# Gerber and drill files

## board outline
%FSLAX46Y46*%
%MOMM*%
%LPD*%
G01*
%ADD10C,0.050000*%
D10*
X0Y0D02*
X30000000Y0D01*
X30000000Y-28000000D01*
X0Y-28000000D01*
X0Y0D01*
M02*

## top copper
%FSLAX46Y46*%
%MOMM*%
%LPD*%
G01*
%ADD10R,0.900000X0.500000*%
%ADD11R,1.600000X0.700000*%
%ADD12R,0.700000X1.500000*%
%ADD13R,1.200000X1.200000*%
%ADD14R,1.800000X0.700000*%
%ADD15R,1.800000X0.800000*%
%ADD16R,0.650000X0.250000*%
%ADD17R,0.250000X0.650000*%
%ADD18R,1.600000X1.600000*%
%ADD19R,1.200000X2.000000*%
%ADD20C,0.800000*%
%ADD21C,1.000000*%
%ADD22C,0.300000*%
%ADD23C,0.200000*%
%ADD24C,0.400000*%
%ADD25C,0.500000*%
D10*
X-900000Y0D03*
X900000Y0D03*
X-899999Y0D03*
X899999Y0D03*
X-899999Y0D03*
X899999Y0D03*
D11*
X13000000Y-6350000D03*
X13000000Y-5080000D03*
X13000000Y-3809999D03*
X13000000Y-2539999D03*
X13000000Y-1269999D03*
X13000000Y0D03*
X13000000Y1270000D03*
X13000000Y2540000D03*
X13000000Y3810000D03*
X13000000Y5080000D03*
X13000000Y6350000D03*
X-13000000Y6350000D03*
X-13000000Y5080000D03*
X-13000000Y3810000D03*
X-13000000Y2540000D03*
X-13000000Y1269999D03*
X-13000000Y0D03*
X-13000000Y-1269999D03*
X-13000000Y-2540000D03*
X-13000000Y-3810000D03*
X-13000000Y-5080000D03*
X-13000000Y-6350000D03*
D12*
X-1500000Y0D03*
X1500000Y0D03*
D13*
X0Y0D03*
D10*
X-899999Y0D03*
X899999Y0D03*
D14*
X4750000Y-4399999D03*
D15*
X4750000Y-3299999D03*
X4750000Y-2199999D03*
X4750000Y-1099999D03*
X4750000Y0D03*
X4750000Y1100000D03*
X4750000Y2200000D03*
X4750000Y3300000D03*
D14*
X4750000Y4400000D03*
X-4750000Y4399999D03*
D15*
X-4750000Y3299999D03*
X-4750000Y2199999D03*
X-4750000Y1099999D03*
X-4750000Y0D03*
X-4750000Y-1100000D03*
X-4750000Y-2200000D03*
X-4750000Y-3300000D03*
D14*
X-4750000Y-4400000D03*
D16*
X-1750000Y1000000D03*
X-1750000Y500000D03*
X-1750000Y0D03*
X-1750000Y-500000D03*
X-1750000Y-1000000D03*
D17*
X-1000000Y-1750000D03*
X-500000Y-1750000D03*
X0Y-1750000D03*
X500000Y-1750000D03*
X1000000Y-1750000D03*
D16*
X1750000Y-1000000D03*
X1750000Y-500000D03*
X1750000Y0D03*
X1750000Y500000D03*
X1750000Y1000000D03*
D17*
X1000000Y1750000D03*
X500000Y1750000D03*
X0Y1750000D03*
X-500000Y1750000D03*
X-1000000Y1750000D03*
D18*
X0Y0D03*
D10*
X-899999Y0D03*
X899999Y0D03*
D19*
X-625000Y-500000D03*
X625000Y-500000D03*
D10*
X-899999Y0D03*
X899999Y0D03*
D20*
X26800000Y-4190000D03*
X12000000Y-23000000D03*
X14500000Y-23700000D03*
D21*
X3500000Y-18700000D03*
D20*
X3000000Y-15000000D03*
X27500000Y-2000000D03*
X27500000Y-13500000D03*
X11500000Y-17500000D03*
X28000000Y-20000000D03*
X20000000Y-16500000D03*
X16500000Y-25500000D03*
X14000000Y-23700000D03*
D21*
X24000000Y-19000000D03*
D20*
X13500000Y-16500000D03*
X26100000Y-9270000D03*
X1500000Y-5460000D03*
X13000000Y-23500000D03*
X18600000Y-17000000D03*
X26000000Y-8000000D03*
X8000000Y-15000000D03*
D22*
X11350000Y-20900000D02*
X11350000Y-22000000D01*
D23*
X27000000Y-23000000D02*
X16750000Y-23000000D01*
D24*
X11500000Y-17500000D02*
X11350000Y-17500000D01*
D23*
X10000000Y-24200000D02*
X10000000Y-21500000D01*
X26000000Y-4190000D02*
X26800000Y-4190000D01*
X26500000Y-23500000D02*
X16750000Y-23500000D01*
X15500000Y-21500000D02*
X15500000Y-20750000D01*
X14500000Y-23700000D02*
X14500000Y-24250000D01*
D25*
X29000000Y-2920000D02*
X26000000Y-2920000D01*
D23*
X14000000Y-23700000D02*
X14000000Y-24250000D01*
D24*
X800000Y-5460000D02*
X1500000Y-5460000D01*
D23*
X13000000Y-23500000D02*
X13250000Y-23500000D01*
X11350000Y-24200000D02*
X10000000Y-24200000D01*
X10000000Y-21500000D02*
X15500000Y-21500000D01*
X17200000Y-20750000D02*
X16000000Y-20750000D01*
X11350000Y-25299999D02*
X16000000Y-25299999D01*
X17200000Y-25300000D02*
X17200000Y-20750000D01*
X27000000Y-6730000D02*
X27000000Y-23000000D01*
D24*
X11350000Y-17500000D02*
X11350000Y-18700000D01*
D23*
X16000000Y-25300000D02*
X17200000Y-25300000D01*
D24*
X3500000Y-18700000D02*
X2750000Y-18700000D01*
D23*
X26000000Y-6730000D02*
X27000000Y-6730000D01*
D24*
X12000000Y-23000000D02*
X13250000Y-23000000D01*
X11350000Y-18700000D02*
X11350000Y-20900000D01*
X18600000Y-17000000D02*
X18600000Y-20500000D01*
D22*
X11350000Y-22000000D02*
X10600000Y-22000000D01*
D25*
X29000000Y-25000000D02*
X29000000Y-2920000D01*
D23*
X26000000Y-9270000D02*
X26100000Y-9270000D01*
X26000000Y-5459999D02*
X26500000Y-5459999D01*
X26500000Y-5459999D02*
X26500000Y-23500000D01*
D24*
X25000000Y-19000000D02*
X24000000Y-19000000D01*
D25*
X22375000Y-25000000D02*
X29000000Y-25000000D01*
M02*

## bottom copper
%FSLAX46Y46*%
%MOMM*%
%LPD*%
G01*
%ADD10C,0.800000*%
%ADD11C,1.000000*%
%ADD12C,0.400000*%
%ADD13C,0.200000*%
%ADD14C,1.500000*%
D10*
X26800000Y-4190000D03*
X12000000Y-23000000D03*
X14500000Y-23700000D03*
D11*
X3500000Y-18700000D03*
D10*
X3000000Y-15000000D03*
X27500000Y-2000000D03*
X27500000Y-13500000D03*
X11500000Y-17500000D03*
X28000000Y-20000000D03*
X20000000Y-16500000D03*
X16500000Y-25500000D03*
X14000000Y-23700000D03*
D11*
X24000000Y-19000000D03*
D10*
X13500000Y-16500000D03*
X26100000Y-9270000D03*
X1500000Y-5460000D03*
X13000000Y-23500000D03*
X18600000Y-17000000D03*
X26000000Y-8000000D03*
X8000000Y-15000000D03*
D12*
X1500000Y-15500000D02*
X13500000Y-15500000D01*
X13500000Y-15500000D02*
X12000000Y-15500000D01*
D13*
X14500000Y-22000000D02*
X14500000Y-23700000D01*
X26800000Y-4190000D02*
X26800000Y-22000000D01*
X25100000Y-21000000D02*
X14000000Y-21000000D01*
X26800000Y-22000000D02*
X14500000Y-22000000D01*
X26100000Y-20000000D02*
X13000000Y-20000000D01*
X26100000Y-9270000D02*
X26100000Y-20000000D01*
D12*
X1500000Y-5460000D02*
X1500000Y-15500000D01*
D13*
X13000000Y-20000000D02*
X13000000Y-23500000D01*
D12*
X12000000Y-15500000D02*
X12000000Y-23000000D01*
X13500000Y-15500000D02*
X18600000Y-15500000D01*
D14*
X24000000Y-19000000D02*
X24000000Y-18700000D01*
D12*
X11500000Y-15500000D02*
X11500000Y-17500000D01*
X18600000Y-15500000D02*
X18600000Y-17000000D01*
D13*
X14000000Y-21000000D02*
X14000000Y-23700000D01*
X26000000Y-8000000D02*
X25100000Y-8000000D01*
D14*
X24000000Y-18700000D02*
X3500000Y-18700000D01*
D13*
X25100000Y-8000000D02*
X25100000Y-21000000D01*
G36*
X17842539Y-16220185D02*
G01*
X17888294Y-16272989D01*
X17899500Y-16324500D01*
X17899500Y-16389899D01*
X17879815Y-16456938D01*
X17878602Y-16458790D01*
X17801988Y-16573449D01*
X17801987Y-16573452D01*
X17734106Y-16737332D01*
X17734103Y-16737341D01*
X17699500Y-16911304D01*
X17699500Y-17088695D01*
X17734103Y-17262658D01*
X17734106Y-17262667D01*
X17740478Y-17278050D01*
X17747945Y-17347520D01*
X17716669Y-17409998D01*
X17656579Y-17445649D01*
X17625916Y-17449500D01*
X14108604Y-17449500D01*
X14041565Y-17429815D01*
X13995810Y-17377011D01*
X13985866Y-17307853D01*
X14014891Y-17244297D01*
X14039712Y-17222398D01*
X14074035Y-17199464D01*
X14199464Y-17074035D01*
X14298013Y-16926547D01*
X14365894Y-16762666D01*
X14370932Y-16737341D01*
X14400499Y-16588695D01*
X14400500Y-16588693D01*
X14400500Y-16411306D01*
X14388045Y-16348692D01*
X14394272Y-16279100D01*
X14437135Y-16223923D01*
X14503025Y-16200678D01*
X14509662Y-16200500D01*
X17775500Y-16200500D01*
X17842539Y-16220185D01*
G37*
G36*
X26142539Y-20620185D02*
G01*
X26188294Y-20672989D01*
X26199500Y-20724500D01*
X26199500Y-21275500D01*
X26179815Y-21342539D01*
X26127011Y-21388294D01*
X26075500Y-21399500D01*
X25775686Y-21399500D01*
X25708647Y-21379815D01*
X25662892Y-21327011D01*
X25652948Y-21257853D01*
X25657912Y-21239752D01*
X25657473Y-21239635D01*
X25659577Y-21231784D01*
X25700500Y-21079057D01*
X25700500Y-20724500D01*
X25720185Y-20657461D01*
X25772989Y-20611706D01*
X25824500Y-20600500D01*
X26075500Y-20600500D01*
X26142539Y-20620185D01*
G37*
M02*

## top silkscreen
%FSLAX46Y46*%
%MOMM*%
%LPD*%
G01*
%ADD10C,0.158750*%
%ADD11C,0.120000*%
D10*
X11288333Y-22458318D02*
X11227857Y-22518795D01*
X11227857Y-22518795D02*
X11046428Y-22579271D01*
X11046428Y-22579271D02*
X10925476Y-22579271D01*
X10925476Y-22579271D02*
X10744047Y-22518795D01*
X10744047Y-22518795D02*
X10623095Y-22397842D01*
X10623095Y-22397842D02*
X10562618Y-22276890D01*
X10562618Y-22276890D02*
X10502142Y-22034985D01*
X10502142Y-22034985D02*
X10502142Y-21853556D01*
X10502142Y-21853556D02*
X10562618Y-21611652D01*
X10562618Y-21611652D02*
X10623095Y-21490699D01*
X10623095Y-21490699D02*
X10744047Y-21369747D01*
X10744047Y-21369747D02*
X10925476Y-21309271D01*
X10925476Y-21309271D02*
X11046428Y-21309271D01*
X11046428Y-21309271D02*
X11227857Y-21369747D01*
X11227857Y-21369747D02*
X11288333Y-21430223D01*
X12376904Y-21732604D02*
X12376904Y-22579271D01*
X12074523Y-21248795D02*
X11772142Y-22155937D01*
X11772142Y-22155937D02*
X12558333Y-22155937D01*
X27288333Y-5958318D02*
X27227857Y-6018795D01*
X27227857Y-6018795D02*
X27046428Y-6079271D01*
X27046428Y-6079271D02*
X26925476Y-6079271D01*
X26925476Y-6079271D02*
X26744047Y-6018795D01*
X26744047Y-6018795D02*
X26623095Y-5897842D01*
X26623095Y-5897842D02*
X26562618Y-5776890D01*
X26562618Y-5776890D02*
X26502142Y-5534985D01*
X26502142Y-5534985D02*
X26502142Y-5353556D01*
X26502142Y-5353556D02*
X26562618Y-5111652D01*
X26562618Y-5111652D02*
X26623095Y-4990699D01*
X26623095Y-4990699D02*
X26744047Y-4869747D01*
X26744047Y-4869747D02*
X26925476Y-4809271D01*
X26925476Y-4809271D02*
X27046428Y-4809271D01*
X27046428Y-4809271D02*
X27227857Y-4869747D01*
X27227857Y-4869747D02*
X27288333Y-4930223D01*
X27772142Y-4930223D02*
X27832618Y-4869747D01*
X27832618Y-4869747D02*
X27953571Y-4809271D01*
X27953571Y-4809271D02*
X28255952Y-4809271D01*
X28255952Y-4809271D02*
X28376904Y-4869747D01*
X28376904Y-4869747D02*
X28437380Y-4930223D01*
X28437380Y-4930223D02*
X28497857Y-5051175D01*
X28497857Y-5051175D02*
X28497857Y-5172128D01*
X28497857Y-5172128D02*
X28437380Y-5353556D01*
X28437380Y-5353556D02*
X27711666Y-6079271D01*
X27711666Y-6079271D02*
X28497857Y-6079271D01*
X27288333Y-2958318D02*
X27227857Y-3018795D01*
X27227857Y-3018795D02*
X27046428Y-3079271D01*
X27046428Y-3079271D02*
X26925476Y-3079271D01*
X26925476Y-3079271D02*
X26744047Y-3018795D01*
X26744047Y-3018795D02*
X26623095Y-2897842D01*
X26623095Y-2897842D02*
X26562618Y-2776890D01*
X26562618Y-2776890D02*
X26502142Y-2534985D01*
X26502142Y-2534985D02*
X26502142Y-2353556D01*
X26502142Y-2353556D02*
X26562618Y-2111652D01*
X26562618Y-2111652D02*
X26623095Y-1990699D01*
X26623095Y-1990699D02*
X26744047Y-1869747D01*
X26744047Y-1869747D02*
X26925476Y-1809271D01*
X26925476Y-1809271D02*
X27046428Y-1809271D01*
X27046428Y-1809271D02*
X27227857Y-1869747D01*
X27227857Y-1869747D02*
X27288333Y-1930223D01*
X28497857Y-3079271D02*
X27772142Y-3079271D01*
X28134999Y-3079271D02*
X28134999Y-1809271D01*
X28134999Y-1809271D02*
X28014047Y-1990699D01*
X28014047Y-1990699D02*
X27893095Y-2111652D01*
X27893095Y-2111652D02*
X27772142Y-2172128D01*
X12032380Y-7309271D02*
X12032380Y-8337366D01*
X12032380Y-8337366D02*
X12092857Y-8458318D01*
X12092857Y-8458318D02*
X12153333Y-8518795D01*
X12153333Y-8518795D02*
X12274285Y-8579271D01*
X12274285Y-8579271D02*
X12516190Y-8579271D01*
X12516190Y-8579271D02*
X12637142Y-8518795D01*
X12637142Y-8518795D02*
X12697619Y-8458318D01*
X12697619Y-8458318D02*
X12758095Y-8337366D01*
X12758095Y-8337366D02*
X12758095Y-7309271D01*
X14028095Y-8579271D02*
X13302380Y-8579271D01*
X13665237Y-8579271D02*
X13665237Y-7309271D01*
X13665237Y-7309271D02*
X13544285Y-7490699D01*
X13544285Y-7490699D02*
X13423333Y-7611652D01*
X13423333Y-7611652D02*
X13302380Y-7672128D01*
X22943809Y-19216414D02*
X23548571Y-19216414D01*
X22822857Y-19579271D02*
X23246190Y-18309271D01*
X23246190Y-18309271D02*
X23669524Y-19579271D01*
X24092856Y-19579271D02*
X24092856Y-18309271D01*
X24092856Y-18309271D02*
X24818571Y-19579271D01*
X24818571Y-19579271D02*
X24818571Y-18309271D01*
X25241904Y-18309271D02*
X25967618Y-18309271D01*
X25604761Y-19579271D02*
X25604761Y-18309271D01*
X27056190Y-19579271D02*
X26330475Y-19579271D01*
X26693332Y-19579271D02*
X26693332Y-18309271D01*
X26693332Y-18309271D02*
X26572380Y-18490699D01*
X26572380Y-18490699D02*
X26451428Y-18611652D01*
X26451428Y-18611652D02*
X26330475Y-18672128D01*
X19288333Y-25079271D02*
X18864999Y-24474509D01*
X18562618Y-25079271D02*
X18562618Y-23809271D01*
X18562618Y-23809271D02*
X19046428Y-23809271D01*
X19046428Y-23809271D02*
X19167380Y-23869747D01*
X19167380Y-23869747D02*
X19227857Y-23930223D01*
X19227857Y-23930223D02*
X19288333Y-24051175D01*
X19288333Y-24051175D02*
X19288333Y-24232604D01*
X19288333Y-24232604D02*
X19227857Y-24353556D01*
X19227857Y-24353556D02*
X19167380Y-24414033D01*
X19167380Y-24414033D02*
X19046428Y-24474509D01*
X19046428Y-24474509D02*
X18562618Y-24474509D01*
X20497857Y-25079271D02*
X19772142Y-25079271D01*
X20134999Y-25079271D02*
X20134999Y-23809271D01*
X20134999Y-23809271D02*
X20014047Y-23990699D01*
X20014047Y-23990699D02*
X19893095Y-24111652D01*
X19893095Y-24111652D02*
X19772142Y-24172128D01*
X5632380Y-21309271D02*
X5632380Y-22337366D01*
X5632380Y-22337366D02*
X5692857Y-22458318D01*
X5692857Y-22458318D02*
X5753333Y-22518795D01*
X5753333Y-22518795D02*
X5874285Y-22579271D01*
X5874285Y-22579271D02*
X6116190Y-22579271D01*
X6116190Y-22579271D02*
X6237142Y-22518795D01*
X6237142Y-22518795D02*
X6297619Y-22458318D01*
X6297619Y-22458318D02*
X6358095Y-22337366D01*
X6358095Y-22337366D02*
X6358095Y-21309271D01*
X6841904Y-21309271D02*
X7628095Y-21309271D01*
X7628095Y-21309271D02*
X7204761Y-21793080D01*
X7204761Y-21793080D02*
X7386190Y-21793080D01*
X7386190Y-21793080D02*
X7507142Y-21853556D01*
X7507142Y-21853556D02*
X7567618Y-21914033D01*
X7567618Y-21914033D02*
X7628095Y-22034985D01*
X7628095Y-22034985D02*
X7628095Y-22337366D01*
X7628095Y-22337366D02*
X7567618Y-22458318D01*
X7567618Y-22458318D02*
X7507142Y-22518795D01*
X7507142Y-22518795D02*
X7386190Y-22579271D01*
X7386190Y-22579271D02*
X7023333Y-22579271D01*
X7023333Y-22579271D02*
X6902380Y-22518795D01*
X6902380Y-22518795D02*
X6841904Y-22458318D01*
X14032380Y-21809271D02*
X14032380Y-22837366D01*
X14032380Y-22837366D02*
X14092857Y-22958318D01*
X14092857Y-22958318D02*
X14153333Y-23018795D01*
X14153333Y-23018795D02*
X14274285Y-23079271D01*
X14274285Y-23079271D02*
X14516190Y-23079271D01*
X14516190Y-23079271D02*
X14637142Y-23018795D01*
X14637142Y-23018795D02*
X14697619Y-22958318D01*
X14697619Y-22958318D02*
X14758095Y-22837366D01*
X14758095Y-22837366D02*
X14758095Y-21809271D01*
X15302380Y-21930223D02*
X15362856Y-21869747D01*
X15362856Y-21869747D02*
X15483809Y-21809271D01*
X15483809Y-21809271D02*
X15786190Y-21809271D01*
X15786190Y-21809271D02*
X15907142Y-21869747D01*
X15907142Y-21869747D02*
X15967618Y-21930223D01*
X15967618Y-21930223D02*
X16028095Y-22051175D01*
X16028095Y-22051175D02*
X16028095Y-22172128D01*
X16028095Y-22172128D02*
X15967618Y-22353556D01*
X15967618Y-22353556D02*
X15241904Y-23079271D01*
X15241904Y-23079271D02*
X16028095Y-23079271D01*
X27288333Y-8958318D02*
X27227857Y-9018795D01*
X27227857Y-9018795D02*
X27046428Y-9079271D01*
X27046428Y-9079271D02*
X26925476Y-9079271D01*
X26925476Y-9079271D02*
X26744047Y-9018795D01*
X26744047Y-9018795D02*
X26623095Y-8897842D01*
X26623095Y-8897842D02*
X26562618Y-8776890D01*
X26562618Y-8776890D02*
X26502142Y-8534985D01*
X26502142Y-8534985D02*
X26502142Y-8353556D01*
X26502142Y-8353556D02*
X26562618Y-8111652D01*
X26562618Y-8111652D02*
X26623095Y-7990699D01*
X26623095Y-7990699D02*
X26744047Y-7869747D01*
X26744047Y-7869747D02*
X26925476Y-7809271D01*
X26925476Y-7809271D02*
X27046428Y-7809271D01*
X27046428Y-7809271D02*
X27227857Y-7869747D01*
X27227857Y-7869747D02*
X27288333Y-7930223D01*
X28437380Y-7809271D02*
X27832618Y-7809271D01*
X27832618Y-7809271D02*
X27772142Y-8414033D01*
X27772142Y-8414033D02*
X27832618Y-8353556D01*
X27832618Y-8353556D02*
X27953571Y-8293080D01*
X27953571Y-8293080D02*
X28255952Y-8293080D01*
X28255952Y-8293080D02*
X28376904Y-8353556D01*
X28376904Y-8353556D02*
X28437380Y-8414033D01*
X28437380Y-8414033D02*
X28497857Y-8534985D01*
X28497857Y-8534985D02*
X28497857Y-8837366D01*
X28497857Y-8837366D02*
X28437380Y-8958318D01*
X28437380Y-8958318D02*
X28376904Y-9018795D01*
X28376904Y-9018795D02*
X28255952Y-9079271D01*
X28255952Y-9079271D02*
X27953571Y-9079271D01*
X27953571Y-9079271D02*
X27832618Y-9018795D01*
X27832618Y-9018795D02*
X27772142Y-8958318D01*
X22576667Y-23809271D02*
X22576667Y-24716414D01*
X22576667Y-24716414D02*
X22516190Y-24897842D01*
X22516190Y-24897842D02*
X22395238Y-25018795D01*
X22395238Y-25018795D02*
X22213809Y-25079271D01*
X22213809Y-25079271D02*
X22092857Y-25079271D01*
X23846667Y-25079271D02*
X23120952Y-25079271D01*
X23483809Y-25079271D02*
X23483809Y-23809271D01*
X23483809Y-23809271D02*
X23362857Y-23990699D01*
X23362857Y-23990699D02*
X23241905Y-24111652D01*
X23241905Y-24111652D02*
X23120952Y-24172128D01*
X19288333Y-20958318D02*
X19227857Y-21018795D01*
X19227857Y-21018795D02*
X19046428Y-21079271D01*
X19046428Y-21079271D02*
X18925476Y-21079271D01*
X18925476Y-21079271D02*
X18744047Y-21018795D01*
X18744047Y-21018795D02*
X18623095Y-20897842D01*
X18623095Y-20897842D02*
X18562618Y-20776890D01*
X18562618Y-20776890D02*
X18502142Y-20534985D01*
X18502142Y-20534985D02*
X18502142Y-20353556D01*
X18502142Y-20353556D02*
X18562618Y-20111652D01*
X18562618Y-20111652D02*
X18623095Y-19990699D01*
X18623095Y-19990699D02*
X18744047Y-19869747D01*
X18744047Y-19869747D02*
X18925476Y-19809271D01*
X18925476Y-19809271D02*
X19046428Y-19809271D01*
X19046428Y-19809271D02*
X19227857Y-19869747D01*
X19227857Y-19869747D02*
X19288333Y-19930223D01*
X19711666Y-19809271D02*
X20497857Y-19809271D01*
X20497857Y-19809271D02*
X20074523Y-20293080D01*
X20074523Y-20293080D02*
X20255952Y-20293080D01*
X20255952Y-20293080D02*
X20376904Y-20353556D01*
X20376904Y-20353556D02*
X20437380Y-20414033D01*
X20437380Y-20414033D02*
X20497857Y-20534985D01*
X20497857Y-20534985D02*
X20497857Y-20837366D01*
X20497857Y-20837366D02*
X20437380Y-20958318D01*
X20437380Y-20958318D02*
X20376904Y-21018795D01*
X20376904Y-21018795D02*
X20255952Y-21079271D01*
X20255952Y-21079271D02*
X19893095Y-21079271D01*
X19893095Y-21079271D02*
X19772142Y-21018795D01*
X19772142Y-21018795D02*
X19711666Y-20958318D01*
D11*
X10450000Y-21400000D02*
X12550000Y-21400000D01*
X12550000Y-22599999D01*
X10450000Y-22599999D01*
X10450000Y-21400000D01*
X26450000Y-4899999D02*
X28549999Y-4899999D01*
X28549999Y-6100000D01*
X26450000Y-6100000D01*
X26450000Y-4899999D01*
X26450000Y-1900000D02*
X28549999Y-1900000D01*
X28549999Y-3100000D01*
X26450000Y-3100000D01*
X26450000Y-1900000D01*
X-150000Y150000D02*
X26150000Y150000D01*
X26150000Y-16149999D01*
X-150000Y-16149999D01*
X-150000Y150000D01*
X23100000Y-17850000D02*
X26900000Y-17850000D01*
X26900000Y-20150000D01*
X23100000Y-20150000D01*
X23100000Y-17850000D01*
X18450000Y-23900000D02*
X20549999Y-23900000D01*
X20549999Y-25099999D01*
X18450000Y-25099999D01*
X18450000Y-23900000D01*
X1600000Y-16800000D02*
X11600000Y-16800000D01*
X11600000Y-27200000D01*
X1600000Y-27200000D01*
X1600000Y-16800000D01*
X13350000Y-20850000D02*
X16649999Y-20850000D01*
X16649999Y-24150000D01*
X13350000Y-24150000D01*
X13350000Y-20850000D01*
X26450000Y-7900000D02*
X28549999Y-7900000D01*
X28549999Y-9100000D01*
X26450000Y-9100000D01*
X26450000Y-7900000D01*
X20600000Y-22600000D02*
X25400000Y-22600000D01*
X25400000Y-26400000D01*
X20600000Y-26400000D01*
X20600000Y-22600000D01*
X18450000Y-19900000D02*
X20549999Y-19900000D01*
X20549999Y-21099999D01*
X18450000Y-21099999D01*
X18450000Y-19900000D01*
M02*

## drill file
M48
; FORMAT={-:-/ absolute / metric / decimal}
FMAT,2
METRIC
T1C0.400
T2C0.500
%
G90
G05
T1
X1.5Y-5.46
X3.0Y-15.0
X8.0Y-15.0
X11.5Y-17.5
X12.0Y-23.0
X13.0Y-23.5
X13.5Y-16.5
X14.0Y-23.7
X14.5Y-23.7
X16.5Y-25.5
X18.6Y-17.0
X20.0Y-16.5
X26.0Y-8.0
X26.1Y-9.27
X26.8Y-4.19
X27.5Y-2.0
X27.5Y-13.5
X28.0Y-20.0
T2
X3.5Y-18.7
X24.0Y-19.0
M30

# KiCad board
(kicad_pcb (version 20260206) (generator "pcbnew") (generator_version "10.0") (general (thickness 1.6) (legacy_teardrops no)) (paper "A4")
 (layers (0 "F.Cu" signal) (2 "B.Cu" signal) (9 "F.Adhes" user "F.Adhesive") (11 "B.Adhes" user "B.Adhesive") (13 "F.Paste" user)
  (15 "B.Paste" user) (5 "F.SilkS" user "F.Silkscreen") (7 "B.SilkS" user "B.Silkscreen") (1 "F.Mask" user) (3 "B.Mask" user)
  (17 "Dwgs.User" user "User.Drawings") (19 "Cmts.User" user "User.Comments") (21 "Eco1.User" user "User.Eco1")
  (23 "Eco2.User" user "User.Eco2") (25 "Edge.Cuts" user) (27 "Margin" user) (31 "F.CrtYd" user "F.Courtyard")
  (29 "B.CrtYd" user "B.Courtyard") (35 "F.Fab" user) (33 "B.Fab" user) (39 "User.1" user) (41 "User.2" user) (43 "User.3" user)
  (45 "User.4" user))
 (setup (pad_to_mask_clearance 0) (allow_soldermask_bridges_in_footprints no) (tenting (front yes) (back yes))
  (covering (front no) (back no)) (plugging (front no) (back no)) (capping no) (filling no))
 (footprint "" (layer "F.Cu") (at 11.5 22)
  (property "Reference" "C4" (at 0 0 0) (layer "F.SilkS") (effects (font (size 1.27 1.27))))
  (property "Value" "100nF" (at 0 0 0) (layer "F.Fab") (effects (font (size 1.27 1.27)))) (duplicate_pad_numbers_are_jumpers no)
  (fp_rect (start -1.05 -0.6) (end 1.05 0.599999) (stroke (width 0.12) (type default)) (fill no) (layer "F.SilkS"))
  (pad "1" smd rect (at -12.4 -22) (size 0.9 0.5) (layers "F.Cu" "F.Mask" "F.Paste") (thermal_bridge_angle 45))
  (pad "2" smd rect (at -10.6 -22) (size 0.9 0.5) (layers "F.Cu" "F.Mask" "F.Paste") (thermal_bridge_angle 45)))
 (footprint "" (layer "F.Cu") (at 27.5 5.5)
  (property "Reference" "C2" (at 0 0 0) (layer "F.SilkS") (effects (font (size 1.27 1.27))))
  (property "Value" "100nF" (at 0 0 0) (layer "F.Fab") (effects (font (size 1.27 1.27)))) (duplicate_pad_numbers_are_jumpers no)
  (fp_rect (start -1.05 -0.600001) (end 1.049999 0.6) (stroke (width 0.12) (type default)) (fill no) (layer "F.SilkS"))
  (pad "1" smd rect (at -28.399999 -5.5) (size 0.9 0.5) (layers "F.Cu" "F.Mask" "F.Paste") (thermal_bridge_angle 45))
  (pad "2" smd rect (at -26.600001 -5.5) (size 0.9 0.5) (layers "F.Cu" "F.Mask" "F.Paste") (thermal_bridge_angle 45)))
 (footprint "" (layer "F.Cu") (at 27.5 2.5)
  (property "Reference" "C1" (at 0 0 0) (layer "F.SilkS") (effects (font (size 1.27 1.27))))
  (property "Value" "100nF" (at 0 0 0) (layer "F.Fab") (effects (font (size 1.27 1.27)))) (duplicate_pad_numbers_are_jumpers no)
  (fp_rect (start -1.05 -0.6) (end 1.049999 0.6) (stroke (width 0.12) (type default)) (fill no) (layer "F.SilkS"))
  (pad "1" smd rect (at -28.399999 -2.5) (size 0.9 0.5) (layers "F.Cu" "F.Mask" "F.Paste") (thermal_bridge_angle 45))
  (pad "2" smd rect (at -26.600001 -2.5) (size 0.9 0.5) (layers "F.Cu" "F.Mask" "F.Paste") (thermal_bridge_angle 45)))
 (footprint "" (layer "F.Cu") (at 13 8)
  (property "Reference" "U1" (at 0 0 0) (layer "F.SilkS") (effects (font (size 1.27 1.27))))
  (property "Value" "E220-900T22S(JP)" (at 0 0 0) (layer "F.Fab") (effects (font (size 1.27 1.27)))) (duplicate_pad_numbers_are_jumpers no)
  (fp_rect (start -13.15 -8.15) (end 13.15 8.149999) (stroke (width 0.12) (type default)) (fill no) (layer "F.SilkS"))
  (pad "1" smd rect (at 0 -1.65) (size 1.6 0.7) (layers "F.Cu" "F.Mask" "F.Paste") (thermal_bridge_angle 45))
  (pad "2" smd rect (at 0 -2.92) (size 1.6 0.7) (layers "F.Cu" "F.Mask" "F.Paste") (thermal_bridge_angle 45))
  (pad "3" smd rect (at 0 -4.190001) (size 1.6 0.7) (layers "F.Cu" "F.Mask" "F.Paste") (thermal_bridge_angle 45))
  (pad "4" smd rect (at 0 -5.460001) (size 1.6 0.7) (layers "F.Cu" "F.Mask" "F.Paste") (thermal_bridge_angle 45))
  (pad "5" smd rect (at 0 -6.730001) (size 1.6 0.7) (layers "F.Cu" "F.Mask" "F.Paste") (thermal_bridge_angle 45))
  (pad "6" smd rect (at 0 -8) (size 1.6 0.7) (layers "F.Cu" "F.Mask" "F.Paste") (thermal_bridge_angle 45))
  (pad "7" smd rect (at 0 -9.27) (size 1.6 0.7) (layers "F.Cu" "F.Mask" "F.Paste") (thermal_bridge_angle 45))
  (pad "8" smd rect (at 0 -10.54) (size 1.6 0.7) (layers "F.Cu" "F.Mask" "F.Paste") (thermal_bridge_angle 45))
  (pad "9" smd rect (at 0 -11.81) (size 1.6 0.7) (layers "F.Cu" "F.Mask" "F.Paste") (thermal_bridge_angle 45))
  (pad "10" smd rect (at 0 -13.08) (size 1.6 0.7) (layers "F.Cu" "F.Mask" "F.Paste") (thermal_bridge_angle 45))
  (pad "11" smd rect (at 0 -14.35) (size 1.6 0.7) (layers "F.Cu" "F.Mask" "F.Paste") (thermal_bridge_angle 45))
  (pad "12" smd rect (at -26 -14.35) (size 1.6 0.7) (layers "F.Cu" "F.Mask" "F.Paste") (thermal_bridge_angle 45))
  (pad "13" smd rect (at -26 -13.08) (size 1.6 0.7) (layers "F.Cu" "F.Mask" "F.Paste") (thermal_bridge_angle 45))
  (pad "14" smd rect (at -26 -11.81) (size 1.6 0.7) (layers "F.Cu" "F.Mask" "F.Paste") (thermal_bridge_angle 45))
  (pad "15" smd rect (at -26 -10.54) (size 1.6 0.7) (layers "F.Cu" "F.Mask" "F.Paste") (thermal_bridge_angle 45))
  (pad "16" smd rect (at -26 -9.269999) (size 1.6 0.7) (layers "F.Cu" "F.Mask" "F.Paste") (thermal_bridge_angle 45))
  (pad "17" smd rect (at -26 -8) (size 1.6 0.7) (layers "F.Cu" "F.Mask" "F.Paste") (thermal_bridge_angle 45))
  (pad "18" smd rect (at -26 -6.730001) (size 1.6 0.7) (layers "F.Cu" "F.Mask" "F.Paste") (thermal_bridge_angle 45))
  (pad "19" smd rect (at -26 -5.46) (size 1.6 0.7) (layers "F.Cu" "F.Mask" "F.Paste") (thermal_bridge_angle 45))
  (pad "20" smd rect (at -26 -4.19) (size 1.6 0.7) (layers "F.Cu" "F.Mask" "F.Paste") (thermal_bridge_angle 45))
  (pad "21" smd rect (at -26 -2.92) (size 1.6 0.7) (layers "F.Cu" "F.Mask" "F.Paste") (thermal_bridge_angle 45))
  (pad "22" smd rect (at -26 -1.65) (size 1.6 0.7) (layers "F.Cu" "F.Mask" "F.Paste") (thermal_bridge_angle 45)))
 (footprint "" (layer "F.Cu") (at 25 19)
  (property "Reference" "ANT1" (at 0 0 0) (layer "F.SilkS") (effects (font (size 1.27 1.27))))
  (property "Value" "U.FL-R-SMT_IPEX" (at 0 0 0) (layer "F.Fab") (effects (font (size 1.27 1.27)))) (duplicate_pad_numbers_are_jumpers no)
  (fp_rect (start -1.9 -1.15) (end 1.9 1.15) (stroke (width 0.12) (type default)) (fill no) (layer "F.SilkS"))
  (pad "G1" smd rect (at -26.5 -19) (size 0.7 1.5) (layers "F.Cu" "F.Mask" "F.Paste") (thermal_bridge_angle 45))
  (pad "G2" smd rect (at -23.5 -19) (size 0.7 1.5) (layers "F.Cu" "F.Mask" "F.Paste") (thermal_bridge_angle 45))
  (pad "S" smd rect (at -25 -19) (size 1.2 1.2) (layers "F.Cu" "F.Mask" "F.Paste") (thermal_bridge_angle 45)))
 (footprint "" (layer "F.Cu") (at 19.5 24.5)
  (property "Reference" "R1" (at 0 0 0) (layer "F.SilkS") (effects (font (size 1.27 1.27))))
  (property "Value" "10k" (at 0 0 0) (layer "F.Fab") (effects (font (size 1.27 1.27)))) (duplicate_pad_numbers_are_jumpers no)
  (fp_rect (start -1.05 -0.6) (end 1.049999 0.599999) (stroke (width 0.12) (type default)) (fill no) (layer "F.SilkS"))
  (pad "1" smd rect (at -20.399999 -24.5) (size 0.9 0.5) (layers "F.Cu" "F.Mask" "F.Paste") (thermal_bridge_angle 45))
  (pad "2" smd rect (at -18.600001 -24.5) (size 0.9 0.5) (layers "F.Cu" "F.Mask" "F.Paste") (thermal_bridge_angle 45)))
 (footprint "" (layer "F.Cu") (at 6.6 22)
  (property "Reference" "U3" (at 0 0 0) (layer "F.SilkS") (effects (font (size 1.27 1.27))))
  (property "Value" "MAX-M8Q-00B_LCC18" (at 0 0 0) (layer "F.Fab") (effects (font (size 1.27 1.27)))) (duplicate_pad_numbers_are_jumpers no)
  (fp_rect (start -5 -5.2) (end 5 5.2) (stroke (width 0.12) (type default)) (fill no) (layer "F.SilkS"))
  (pad "1" smd rect (at -1.85 -17.600001) (size 1.8 0.7) (layers "F.Cu" "F.Mask" "F.Paste") (thermal_bridge_angle 45))
  (pad "2" smd rect (at -1.85 -18.700001) (size 1.8 0.8) (layers "F.Cu" "F.Mask" "F.Paste") (thermal_bridge_angle 45))
  (pad "3" smd rect (at -1.85 -19.800001) (size 1.8 0.8) (layers "F.Cu" "F.Mask" "F.Paste") (thermal_bridge_angle 45))
  (pad "4" smd rect (at -1.85 -20.900001) (size 1.8 0.8) (layers "F.Cu" "F.Mask" "F.Paste") (thermal_bridge_angle 45))
  (pad "5" smd rect (at -1.85 -22) (size 1.8 0.8) (layers "F.Cu" "F.Mask" "F.Paste") (thermal_bridge_angle 45))
  (pad "6" smd rect (at -1.85 -23.1) (size 1.8 0.8) (layers "F.Cu" "F.Mask" "F.Paste") (thermal_bridge_angle 45))
  (pad "7" smd rect (at -1.85 -24.2) (size 1.8 0.8) (layers "F.Cu" "F.Mask" "F.Paste") (thermal_bridge_angle 45))
  (pad "8" smd rect (at -1.85 -25.3) (size 1.8 0.8) (layers "F.Cu" "F.Mask" "F.Paste") (thermal_bridge_angle 45))
  (pad "9" smd rect (at -1.85 -26.4) (size 1.8 0.7) (layers "F.Cu" "F.Mask" "F.Paste") (thermal_bridge_angle 45))
  (pad "10" smd rect (at -11.35 -26.399999) (size 1.8 0.7) (layers "F.Cu" "F.Mask" "F.Paste") (thermal_bridge_angle 45))
  (pad "11" smd rect (at -11.35 -25.299999) (size 1.8 0.8) (layers "F.Cu" "F.Mask" "F.Paste") (thermal_bridge_angle 45))
  (pad "12" smd rect (at -11.35 -24.199999) (size 1.8 0.8) (layers "F.Cu" "F.Mask" "F.Paste") (thermal_bridge_angle 45))
  (pad "13" smd rect (at -11.35 -23.099999) (size 1.8 0.8) (layers "F.Cu" "F.Mask" "F.Paste") (thermal_bridge_angle 45))
  (pad "14" smd rect (at -11.35 -22) (size 1.8 0.8) (layers "F.Cu" "F.Mask" "F.Paste") (thermal_bridge_angle 45))
  (pad "15" smd rect (at -11.35 -20.9) (size 1.8 0.8) (layers "F.Cu" "F.Mask" "F.Paste") (thermal_bridge_angle 45))
  (pad "16" smd rect (at -11.35 -19.8) (size 1.8 0.8) (layers "F.Cu" "F.Mask" "F.Paste") (thermal_bridge_angle 45))
  (pad "17" smd rect (at -11.35 -18.7) (size 1.8 0.8) (layers "F.Cu" "F.Mask" "F.Paste") (thermal_bridge_angle 45))
  (pad "18" smd rect (at -11.35 -17.6) (size 1.8 0.7) (layers "F.Cu" "F.Mask" "F.Paste") (thermal_bridge_angle 45)))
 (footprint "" (layer "F.Cu") (at 15 22.5)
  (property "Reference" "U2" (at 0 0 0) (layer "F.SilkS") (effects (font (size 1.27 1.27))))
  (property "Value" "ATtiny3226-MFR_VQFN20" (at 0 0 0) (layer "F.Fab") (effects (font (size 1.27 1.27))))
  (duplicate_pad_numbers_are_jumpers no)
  (fp_rect (start -1.65 -1.65) (end 1.649999 1.65) (stroke (width 0.12) (type default)) (fill no) (layer "F.SilkS"))
  (pad "1" smd rect (at -16.75 -23.5) (size 0.65 0.25) (layers "F.Cu" "F.Mask" "F.Paste") (thermal_bridge_angle 45))
  (pad "2" smd rect (at -16.75 -23) (size 0.65 0.25) (layers "F.Cu" "F.Mask" "F.Paste") (thermal_bridge_angle 45))
  (pad "3" smd rect (at -16.75 -22.5) (size 0.65 0.25) (layers "F.Cu" "F.Mask" "F.Paste") (thermal_bridge_angle 45))
  (pad "4" smd rect (at -16.75 -22) (size 0.65 0.25) (layers "F.Cu" "F.Mask" "F.Paste") (thermal_bridge_angle 45))
  (pad "5" smd rect (at -16.75 -21.5) (size 0.65 0.25) (layers "F.Cu" "F.Mask" "F.Paste") (thermal_bridge_angle 45))
  (pad "6" smd rect (at -16 -20.75) (size 0.25 0.65) (layers "F.Cu" "F.Mask" "F.Paste") (thermal_bridge_angle 45))
  (pad "7" smd rect (at -15.5 -20.75) (size 0.25 0.65) (layers "F.Cu" "F.Mask" "F.Paste") (thermal_bridge_angle 45))
  (pad "8" smd rect (at -15 -20.75) (size 0.25 0.65) (layers "F.Cu" "F.Mask" "F.Paste") (thermal_bridge_angle 45))
  (pad "9" smd rect (at -14.5 -20.75) (size 0.25 0.65) (layers "F.Cu" "F.Mask" "F.Paste") (thermal_bridge_angle 45))
  (pad "10" smd rect (at -14 -20.75) (size 0.25 0.65) (layers "F.Cu" "F.Mask" "F.Paste") (thermal_bridge_angle 45))
  (pad "11" smd rect (at -13.25 -21.5) (size 0.65 0.25) (layers "F.Cu" "F.Mask" "F.Paste") (thermal_bridge_angle 45))
  (pad "12" smd rect (at -13.25 -22) (size 0.65 0.25) (layers "F.Cu" "F.Mask" "F.Paste") (thermal_bridge_angle 45))
  (pad "13" smd rect (at -13.25 -22.5) (size 0.65 0.25) (layers "F.Cu" "F.Mask" "F.Paste") (thermal_bridge_angle 45))
  (pad "14" smd rect (at -13.25 -23) (size 0.65 0.25) (layers "F.Cu" "F.Mask" "F.Paste") (thermal_bridge_angle 45))
  (pad "15" smd rect (at -13.25 -23.5) (size 0.65 0.25) (layers "F.Cu" "F.Mask" "F.Paste") (thermal_bridge_angle 45))
  (pad "16" smd rect (at -14 -24.25) (size 0.25 0.65) (layers "F.Cu" "F.Mask" "F.Paste") (thermal_bridge_angle 45))
  (pad "17" smd rect (at -14.5 -24.25) (size 0.25 0.65) (layers "F.Cu" "F.Mask" "F.Paste") (thermal_bridge_angle 45))
  (pad "18" smd rect (at -15 -24.25) (size 0.25 0.65) (layers "F.Cu" "F.Mask" "F.Paste") (thermal_bridge_angle 45))
  (pad "19" smd rect (at -15.5 -24.25) (size 0.25 0.65) (layers "F.Cu" "F.Mask" "F.Paste") (thermal_bridge_angle 45))
  (pad "20" smd rect (at -16 -24.25) (size 0.25 0.65) (layers "F.Cu" "F.Mask" "F.Paste") (thermal_bridge_angle 45))
  (pad "EP" smd rect (at -15 -22.5) (size 1.6 1.6) (layers "F.Cu" "F.Mask" "F.Paste") (thermal_bridge_angle 45)))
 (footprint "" (layer "F.Cu") (at 27.5 8.5)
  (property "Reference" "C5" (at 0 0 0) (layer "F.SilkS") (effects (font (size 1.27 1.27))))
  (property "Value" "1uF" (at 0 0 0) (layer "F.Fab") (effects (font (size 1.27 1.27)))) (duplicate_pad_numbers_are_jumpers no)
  (fp_rect (start -1.05 -0.6) (end 1.049999 0.6) (stroke (width 0.12) (type default)) (fill no) (layer "F.SilkS"))
  (pad "1" smd rect (at -28.399999 -8.5) (size 0.9 0.5) (layers "F.Cu" "F.Mask" "F.Paste") (thermal_bridge_angle 45))
  (pad "2" smd rect (at -26.600001 -8.5) (size 0.9 0.5) (layers "F.Cu" "F.Mask" "F.Paste") (thermal_bridge_angle 45)))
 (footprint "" (layer "F.Cu") (at 23 24.5)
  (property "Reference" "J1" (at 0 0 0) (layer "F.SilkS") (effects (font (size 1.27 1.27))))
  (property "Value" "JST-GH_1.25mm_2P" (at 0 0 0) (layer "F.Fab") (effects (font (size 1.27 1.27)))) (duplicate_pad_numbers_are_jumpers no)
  (fp_rect (start -2.4 -1.9) (end 2.4 1.9) (stroke (width 0.12) (type default)) (fill no) (layer "F.SilkS"))
  (pad "1" smd rect (at -23.625 -24) (size 1.2 2) (layers "F.Cu" "F.Mask" "F.Paste") (thermal_bridge_angle 45))
  (pad "2" smd rect (at -22.375 -24) (size 1.2 2) (layers "F.Cu" "F.Mask" "F.Paste") (thermal_bridge_angle 45)))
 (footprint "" (layer "F.Cu") (at 19.5 20.5)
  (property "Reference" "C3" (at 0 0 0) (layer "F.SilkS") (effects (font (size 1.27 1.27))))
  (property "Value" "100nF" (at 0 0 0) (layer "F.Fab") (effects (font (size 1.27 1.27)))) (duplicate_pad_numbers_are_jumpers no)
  (fp_rect (start -1.05 -0.6) (end 1.049999 0.599999) (stroke (width 0.12) (type default)) (fill no) (layer "F.SilkS"))
  (pad "1" smd rect (at -20.399999 -20.5) (size 0.9 0.5) (layers "F.Cu" "F.Mask" "F.Paste") (thermal_bridge_angle 45))
  (pad "2" smd rect (at -18.600001 -20.5) (size 0.9 0.5) (layers "F.Cu" "F.Mask" "F.Paste") (thermal_bridge_angle 45)))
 (gr_rect (start 0 0) (end 30 28) (stroke (width 0.05) (type default)) (fill no) (layer "Edge.Cuts"))
 (segment (start 11.35 20.9) (end 11.35 22) (width 0.3) (layer "F.Cu") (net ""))
 (segment (start 27 23) (end 16.75 23) (width 0.2) (layer "F.Cu") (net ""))
 (segment (start 11.5 17.5) (end 11.35 17.5) (width 0.4) (layer "F.Cu") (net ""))
 (segment (start 10 24.2) (end 10 21.5) (width 0.2) (layer "F.Cu") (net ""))
 (segment (start 26 4.19) (end 26.8 4.19) (width 0.2) (layer "F.Cu") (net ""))
 (segment (start 26.5 23.5) (end 16.75 23.5) (width 0.2) (layer "F.Cu") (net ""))
 (segment (start 15.5 21.5) (end 15.5 20.75) (width 0.2) (layer "F.Cu") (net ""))
 (segment (start 14.5 23.7) (end 14.5 24.25) (width 0.2) (layer "F.Cu") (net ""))
 (segment (start 29 2.92) (end 26 2.92) (width 0.5) (layer "F.Cu") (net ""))
 (segment (start 14 23.7) (end 14 24.25) (width 0.2) (layer "F.Cu") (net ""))
 (segment (start 0.8 5.46) (end 1.5 5.46) (width 0.4) (layer "F.Cu") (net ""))
 (segment (start 13 23.5) (end 13.25 23.5) (width 0.2) (layer "F.Cu") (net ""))
 (segment (start 11.35 24.2) (end 10 24.2) (width 0.2) (layer "F.Cu") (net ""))
 (segment (start 10 21.5) (end 15.5 21.5) (width 0.2) (layer "F.Cu") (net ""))
 (segment (start 17.2 20.75) (end 16 20.75) (width 0.2) (layer "F.Cu") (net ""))
 (segment (start 11.35 25.299999) (end 16 25.299999) (width 0.2) (layer "F.Cu") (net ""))
 (segment (start 17.2 25.3) (end 17.2 20.75) (width 0.2) (layer "F.Cu") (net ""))
 (segment (start 27 6.73) (end 27 23) (width 0.2) (layer "F.Cu") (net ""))
 (segment (start 11.35 17.5) (end 11.35 18.7) (width 0.4) (layer "F.Cu") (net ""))
 (segment (start 16 25.3) (end 17.2 25.3) (width 0.2) (layer "F.Cu") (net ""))
 (segment (start 3.5 18.7) (end 2.75 18.7) (width 0.4) (layer "F.Cu") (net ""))
 (segment (start 26 6.73) (end 27 6.73) (width 0.2) (layer "F.Cu") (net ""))
 (segment (start 12 23) (end 13.25 23) (width 0.4) (layer "F.Cu") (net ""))
 (segment (start 11.35 18.7) (end 11.35 20.9) (width 0.4) (layer "F.Cu") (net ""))
 (segment (start 18.6 17) (end 18.6 20.5) (width 0.4) (layer "F.Cu") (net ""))
 (segment (start 11.35 22) (end 10.6 22) (width 0.3) (layer "F.Cu") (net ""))
 (segment (start 29 25) (end 29 2.92) (width 0.5) (layer "F.Cu") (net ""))
 (segment (start 26 9.27) (end 26.1 9.27) (width 0.2) (layer "F.Cu") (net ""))
 (segment (start 26 5.459999) (end 26.5 5.459999) (width 0.2) (layer "F.Cu") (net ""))
 (segment (start 26.5 5.459999) (end 26.5 23.5) (width 0.2) (layer "F.Cu") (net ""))
 (segment (start 25 19) (end 24 19) (width 0.4) (layer "F.Cu") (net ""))
 (segment (start 22.375 25) (end 29 25) (width 0.5) (layer "F.Cu") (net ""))
 (via (at 26.8 4.19) (size 0.8) (drill 0.4) (layers "F.Cu" "B.Cu") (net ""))
 (via (at 12 23) (size 0.8) (drill 0.4) (layers "F.Cu" "B.Cu") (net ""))
 (via (at 14.5 23.7) (size 0.8) (drill 0.4) (layers "F.Cu" "B.Cu") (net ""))
 (via (at 3.5 18.7) (size 1) (drill 0.5) (layers "F.Cu" "B.Cu") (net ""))
 (via (at 3 15) (size 0.8) (drill 0.4) (layers "F.Cu" "B.Cu") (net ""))
 (via (at 27.5 2) (size 0.8) (drill 0.4) (layers "F.Cu" "B.Cu") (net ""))
 (via (at 27.5 13.5) (size 0.8) (drill 0.4) (layers "F.Cu" "B.Cu") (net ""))
 (via (at 11.5 17.5) (size 0.8) (drill 0.4) (layers "F.Cu" "B.Cu") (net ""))
 (via (at 28 20) (size 0.8) (drill 0.4) (layers "F.Cu" "B.Cu") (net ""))
 (via (at 20 16.5) (size 0.8) (drill 0.4) (layers "F.Cu" "B.Cu") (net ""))
 (via (at 16.5 25.5) (size 0.8) (drill 0.4) (layers "F.Cu" "B.Cu") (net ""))
 (via (at 14 23.7) (size 0.8) (drill 0.4) (layers "F.Cu" "B.Cu") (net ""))
 (via (at 24 19) (size 1) (drill 0.5) (layers "F.Cu" "B.Cu") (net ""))
 (via (at 13.5 16.5) (size 0.8) (drill 0.4) (layers "F.Cu" "B.Cu") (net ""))
 (via (at 26.1 9.27) (size 0.8) (drill 0.4) (layers "F.Cu" "B.Cu") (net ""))
 (via (at 1.5 5.46) (size 0.8) (drill 0.4) (layers "F.Cu" "B.Cu") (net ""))
 (via (at 13 23.5) (size 0.8) (drill 0.4) (layers "F.Cu" "B.Cu") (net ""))
 (via (at 18.6 17) (size 0.8) (drill 0.4) (layers "F.Cu" "B.Cu") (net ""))
 (via (at 26 8) (size 0.8) (drill 0.4) (layers "F.Cu" "B.Cu") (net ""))
 (via (at 8 15) (size 0.8) (drill 0.4) (layers "F.Cu" "B.Cu") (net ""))
 (segment (start 1.5 15.5) (end 13.5 15.5) (width 0.4) (layer "B.Cu") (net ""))
 (segment (start 13.5 15.5) (end 12 15.5) (width 0.4) (layer "B.Cu") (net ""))
 (segment (start 14.5 22) (end 14.5 23.7) (width 0.2) (layer "B.Cu") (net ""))
 (segment (start 26.8 4.19) (end 26.8 22) (width 0.2) (layer "B.Cu") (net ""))
 (segment (start 25.1 21) (end 14 21) (width 0.2) (layer "B.Cu") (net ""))
 (segment (start 26.8 22) (end 14.5 22) (width 0.2) (layer "B.Cu") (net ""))
 (segment (start 26.1 20) (end 13 20) (width 0.2) (layer "B.Cu") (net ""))
 (segment (start 26.1 9.27) (end 26.1 20) (width 0.2) (layer "B.Cu") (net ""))
 (segment (start 1.5 5.46) (end 1.5 15.5) (width 0.4) (layer "B.Cu") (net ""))
 (segment (start 13 20) (end 13 23.5) (width 0.2) (layer "B.Cu") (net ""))
 (segment (start 12 15.5) (end 12 23) (width 0.4) (layer "B.Cu") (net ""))
 (segment (start 13.5 15.5) (end 18.6 15.5) (width 0.4) (layer "B.Cu") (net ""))
 (segment (start 24 19) (end 24 18.7) (width 1.5) (layer "B.Cu") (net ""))
 (segment (start 11.5 15.5) (end 11.5 17.5) (width 0.4) (layer "B.Cu") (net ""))
 (segment (start 18.6 15.5) (end 18.6 17) (width 0.4) (layer "B.Cu") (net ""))
 (segment (start 14 21) (end 14 23.7) (width 0.2) (layer "B.Cu") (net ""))
 (segment (start 26 8) (end 25.1 8) (width 0.2) (layer "B.Cu") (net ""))
 (segment (start 24 18.7) (end 3.5 18.7) (width 1.5) (layer "B.Cu") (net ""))
 (segment (start 25.1 8) (end 25.1 21) (width 0.2) (layer "B.Cu") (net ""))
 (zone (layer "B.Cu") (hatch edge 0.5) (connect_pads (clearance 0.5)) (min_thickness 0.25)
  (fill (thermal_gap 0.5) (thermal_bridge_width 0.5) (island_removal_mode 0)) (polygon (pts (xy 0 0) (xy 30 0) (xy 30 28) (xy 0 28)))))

